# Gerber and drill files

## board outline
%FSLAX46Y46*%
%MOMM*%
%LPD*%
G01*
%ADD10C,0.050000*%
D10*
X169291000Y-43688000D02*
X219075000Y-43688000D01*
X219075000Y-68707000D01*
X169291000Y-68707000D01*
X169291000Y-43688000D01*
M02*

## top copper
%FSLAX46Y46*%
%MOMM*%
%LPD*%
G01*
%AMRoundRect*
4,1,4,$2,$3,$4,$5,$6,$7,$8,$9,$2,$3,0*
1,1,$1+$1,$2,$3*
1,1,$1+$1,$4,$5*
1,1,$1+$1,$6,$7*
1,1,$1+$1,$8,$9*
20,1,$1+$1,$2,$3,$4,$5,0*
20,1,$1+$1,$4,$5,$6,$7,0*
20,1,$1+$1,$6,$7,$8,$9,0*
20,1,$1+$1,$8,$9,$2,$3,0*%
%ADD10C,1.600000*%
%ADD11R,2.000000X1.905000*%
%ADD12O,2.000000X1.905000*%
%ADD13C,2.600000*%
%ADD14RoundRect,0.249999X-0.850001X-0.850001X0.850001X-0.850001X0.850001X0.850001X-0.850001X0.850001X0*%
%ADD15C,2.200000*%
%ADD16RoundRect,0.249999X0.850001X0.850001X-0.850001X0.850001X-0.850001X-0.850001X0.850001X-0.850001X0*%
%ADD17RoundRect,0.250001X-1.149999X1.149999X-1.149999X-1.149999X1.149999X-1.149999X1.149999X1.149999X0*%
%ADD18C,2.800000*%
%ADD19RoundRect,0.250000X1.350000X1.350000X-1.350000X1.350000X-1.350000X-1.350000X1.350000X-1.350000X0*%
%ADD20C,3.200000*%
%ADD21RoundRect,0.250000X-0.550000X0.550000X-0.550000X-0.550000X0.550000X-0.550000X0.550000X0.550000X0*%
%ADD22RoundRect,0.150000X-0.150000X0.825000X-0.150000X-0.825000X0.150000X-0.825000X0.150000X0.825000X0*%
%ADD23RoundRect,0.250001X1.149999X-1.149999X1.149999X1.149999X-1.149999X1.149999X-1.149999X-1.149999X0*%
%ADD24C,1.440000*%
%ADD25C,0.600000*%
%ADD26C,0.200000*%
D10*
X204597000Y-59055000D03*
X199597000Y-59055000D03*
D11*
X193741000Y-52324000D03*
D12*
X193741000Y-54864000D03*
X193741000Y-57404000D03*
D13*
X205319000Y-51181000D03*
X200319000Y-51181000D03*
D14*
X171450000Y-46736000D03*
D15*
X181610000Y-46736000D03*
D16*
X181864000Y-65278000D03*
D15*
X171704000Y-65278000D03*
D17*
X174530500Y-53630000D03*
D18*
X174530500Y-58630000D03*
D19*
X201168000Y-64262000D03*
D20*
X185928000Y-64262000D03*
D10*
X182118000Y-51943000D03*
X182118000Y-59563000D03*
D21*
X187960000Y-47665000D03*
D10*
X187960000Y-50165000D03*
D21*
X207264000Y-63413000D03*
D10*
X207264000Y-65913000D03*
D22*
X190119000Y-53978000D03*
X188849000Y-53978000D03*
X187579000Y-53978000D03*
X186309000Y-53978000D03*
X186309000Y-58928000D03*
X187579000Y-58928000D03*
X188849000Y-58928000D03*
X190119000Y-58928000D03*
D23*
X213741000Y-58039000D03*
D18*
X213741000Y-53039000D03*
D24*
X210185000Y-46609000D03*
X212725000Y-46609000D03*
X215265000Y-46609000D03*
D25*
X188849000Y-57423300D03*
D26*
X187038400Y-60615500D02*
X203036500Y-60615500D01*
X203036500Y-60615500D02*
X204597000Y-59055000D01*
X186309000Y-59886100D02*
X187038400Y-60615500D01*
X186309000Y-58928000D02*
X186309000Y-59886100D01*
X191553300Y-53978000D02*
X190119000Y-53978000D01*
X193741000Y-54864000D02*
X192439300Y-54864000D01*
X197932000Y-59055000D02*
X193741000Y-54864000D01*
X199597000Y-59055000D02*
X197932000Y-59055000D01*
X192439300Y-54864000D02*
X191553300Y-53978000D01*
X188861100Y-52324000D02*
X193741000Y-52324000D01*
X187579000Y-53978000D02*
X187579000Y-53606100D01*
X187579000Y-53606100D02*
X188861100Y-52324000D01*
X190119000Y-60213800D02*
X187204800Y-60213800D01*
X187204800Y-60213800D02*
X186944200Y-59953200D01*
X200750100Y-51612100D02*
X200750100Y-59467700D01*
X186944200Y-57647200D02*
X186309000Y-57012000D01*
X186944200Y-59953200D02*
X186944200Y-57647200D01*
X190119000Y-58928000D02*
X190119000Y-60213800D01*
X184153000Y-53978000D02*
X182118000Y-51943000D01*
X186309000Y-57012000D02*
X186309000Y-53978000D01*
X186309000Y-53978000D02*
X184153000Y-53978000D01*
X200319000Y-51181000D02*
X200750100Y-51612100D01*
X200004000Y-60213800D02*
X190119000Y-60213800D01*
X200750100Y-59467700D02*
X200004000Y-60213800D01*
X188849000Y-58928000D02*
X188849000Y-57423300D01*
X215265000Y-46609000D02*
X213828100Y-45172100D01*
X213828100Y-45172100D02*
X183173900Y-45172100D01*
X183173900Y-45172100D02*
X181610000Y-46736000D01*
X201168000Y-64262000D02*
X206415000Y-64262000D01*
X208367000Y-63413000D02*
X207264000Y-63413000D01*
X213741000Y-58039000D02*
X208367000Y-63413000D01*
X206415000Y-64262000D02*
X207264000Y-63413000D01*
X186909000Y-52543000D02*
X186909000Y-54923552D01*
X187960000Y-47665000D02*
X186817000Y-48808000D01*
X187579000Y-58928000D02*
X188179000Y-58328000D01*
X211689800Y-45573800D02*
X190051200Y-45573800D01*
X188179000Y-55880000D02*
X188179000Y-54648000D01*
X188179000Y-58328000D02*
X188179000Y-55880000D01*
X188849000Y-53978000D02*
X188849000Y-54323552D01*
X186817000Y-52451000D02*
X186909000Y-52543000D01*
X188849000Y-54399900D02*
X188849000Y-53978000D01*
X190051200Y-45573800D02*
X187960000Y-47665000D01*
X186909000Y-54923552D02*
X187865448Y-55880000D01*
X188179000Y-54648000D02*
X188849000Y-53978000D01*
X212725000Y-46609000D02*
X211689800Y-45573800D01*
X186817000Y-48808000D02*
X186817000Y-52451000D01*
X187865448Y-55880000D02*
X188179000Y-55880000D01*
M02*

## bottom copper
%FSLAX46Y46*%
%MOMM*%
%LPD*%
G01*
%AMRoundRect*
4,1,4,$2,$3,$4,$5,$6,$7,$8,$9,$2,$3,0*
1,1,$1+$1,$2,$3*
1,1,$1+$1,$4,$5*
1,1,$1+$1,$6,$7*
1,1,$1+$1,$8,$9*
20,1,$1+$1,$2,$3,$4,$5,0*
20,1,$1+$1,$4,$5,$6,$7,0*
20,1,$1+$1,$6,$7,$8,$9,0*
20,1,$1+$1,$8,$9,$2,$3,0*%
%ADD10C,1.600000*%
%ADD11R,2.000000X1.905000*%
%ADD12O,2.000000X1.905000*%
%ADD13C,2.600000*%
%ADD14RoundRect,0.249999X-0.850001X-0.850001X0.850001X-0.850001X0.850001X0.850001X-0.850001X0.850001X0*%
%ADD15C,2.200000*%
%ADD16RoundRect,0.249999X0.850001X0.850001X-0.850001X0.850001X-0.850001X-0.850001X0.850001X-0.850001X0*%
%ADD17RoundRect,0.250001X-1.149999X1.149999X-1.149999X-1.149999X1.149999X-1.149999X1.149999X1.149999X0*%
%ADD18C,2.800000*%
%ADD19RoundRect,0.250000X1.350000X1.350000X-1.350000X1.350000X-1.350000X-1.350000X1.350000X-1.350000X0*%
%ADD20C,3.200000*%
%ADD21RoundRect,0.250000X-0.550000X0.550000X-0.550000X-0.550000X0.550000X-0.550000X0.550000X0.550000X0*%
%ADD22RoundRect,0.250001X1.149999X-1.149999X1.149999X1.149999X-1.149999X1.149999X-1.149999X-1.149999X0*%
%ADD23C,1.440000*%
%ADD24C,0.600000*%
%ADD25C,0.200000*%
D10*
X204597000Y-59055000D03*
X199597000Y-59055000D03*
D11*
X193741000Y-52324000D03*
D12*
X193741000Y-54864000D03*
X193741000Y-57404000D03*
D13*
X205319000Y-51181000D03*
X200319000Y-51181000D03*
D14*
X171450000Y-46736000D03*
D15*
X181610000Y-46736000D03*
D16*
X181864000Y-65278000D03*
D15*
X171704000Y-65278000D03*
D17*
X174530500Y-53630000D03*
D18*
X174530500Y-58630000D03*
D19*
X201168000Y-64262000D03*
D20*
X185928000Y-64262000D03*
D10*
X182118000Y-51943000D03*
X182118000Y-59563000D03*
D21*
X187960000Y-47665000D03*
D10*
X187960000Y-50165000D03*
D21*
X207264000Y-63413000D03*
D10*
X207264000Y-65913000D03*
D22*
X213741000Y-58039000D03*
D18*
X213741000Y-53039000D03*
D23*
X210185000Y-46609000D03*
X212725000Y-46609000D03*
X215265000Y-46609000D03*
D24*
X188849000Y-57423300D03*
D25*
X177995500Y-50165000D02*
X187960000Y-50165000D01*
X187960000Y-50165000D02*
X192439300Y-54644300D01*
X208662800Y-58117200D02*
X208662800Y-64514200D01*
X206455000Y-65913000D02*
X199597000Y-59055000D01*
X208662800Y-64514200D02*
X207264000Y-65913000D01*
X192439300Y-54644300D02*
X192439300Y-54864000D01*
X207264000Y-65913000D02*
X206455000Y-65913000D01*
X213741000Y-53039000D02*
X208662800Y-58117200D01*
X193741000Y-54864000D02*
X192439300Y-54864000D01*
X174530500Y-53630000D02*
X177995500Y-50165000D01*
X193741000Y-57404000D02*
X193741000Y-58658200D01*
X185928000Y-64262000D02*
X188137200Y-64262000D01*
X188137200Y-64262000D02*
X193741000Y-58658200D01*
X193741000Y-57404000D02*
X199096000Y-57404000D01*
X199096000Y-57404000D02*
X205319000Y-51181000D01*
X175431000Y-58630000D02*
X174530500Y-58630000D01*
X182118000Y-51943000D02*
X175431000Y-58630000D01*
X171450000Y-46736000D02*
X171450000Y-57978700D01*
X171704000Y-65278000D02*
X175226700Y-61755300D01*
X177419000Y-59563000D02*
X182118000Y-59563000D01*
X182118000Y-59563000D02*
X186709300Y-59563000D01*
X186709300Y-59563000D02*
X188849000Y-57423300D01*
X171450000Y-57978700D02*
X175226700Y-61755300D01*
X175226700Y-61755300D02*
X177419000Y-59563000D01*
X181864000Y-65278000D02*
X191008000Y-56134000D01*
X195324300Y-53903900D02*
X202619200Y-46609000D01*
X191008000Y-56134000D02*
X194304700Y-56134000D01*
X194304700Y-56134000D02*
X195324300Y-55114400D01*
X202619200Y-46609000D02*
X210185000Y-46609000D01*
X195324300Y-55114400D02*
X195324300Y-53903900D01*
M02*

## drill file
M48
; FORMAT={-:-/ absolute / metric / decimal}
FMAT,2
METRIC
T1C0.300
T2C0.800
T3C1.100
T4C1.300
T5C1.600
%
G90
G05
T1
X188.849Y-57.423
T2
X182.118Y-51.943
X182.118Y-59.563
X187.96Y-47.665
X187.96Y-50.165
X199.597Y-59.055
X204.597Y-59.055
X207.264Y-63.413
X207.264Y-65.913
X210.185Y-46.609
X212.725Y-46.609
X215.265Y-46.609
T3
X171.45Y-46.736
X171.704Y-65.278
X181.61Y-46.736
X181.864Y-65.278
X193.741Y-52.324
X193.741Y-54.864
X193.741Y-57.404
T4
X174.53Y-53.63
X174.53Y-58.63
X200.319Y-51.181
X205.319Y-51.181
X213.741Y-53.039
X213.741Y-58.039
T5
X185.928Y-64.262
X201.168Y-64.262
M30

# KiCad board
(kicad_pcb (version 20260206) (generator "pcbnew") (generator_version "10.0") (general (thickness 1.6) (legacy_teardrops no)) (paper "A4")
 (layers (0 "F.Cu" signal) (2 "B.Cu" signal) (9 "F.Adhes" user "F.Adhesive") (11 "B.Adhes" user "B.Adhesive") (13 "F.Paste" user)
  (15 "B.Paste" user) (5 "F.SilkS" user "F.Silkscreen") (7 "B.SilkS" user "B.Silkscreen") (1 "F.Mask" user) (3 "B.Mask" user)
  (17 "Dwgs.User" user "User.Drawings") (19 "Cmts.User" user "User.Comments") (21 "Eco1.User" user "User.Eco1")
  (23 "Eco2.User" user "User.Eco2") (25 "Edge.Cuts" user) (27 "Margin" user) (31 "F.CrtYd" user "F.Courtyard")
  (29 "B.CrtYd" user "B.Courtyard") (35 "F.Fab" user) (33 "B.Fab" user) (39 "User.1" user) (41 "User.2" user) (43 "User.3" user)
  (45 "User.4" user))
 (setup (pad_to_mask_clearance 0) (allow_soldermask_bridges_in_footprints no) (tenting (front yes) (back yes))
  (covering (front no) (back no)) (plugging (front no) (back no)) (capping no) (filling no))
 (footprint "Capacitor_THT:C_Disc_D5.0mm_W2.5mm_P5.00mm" (layer "F.Cu") (at 204.597 59.055 180)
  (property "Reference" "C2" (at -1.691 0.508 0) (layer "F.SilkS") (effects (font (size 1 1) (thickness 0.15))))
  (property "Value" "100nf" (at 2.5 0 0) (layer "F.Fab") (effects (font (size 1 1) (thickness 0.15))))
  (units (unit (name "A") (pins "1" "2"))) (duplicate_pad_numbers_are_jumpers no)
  (pad "1" thru_hole circle (at 0 0 180) (size 1.6 1.6) (drill 0.8) (layers "*.Cu" "*.Mask") (remove_unused_layers no) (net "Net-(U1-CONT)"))
  (pad "2" thru_hole circle (at 5 0 180) (size 1.6 1.6) (drill 0.8) (layers "*.Cu" "*.Mask") (remove_unused_layers no) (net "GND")))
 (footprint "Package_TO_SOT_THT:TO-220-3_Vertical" (layer "F.Cu") (at 193.741 52.324 -90)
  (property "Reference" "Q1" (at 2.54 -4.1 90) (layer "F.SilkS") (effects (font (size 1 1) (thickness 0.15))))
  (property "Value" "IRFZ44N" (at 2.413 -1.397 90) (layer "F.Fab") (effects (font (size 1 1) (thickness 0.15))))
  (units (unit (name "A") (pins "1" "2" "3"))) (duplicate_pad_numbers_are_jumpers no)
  (pad "1" thru_hole rect (at 0 0 270) (size 1.905 2) (drill 1.1) (layers "*.Cu" "*.Mask") (remove_unused_layers no) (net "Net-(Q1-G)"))
  (pad "2" thru_hole oval (at 2.54 0 270) (size 1.905 2) (drill 1.1) (layers "*.Cu" "*.Mask") (remove_unused_layers no) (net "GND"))
  (pad "3" thru_hole oval (at 5.08 0 270) (size 1.905 2) (drill 1.1) (layers "*.Cu" "*.Mask") (remove_unused_layers no) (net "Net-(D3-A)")))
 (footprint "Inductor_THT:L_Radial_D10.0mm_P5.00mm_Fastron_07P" (layer "F.Cu") (at 205.319 51.181 180)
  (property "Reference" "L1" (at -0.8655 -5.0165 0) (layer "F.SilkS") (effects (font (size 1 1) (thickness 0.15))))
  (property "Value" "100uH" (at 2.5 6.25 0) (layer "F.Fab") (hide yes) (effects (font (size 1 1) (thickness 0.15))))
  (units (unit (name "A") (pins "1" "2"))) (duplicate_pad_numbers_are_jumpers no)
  (pad "1" thru_hole circle (at 0 0 180) (size 2.6 2.6) (drill 1.3) (layers "*.Cu" "*.Mask") (remove_unused_layers no) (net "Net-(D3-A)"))
  (pad "2" thru_hole circle (at 5 0 180) (size 2.6 2.6) (drill 1.3) (layers "*.Cu" "*.Mask") (remove_unused_layers no)
   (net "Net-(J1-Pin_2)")))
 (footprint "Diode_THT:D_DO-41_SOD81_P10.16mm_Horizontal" (layer "F.Cu") (at 171.45 46.736)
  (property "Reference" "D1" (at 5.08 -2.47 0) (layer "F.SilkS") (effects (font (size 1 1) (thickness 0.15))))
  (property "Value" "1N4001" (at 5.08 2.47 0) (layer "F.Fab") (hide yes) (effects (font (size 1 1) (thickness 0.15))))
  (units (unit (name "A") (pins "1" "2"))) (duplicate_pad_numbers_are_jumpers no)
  (pad "1" thru_hole roundrect (at 0 0) (size 2.2 2.2) (drill 1.1) (layers "*.Cu" "*.Mask") (remove_unused_layers no)
   (roundrect_rratio 0.113636) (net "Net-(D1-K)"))
  (pad "2" thru_hole circle (at 10.16 0) (size 2.2 2.2) (drill 1.1) (layers "*.Cu" "*.Mask") (remove_unused_layers no) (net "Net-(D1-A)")))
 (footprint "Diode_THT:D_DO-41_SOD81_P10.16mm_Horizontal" (layer "F.Cu") (at 181.864 65.278 180)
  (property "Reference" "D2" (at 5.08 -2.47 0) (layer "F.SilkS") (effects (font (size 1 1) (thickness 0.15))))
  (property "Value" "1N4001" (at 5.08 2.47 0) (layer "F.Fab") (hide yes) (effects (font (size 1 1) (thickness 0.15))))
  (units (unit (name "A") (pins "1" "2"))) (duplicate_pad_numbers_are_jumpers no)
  (pad "1" thru_hole roundrect (at 0 0 180) (size 2.2 2.2) (drill 1.1) (layers "*.Cu" "*.Mask") (remove_unused_layers no)
   (roundrect_rratio 0.113636) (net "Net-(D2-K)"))
  (pad "2" thru_hole circle (at 10.16 0 180) (size 2.2 2.2) (drill 1.1) (layers "*.Cu" "*.Mask") (remove_unused_layers no)
   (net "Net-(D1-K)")))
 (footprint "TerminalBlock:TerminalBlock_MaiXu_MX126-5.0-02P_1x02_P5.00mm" (layer "F.Cu") (at 174.5305 53.63 -90)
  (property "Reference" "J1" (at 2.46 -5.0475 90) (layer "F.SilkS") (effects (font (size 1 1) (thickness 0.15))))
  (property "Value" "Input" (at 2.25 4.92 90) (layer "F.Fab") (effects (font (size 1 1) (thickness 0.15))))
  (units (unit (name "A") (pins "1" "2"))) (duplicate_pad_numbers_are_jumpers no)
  (pad "1" thru_hole roundrect (at 0 0 270) (size 2.8 2.8) (drill 1.3) (layers "*.Cu" "*.Mask") (remove_unused_layers no)
   (roundrect_rratio 0.089286) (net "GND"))
  (pad "2" thru_hole circle (at 5 0 270) (size 2.8 2.8) (drill 1.3) (layers "*.Cu" "*.Mask") (remove_unused_layers no)
   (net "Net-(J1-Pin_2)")))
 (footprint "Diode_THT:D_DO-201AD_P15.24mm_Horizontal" (layer "F.Cu") (at 201.168 64.262 180)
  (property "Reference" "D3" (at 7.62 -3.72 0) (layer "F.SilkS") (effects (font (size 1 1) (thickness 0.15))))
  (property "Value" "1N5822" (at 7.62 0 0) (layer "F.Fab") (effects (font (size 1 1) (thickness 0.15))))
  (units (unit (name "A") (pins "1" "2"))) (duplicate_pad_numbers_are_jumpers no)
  (pad "1" thru_hole roundrect (at 0 0 180) (size 3.2 3.2) (drill 1.6) (layers "*.Cu" "*.Mask") (remove_unused_layers no)
   (roundrect_rratio 0.078125) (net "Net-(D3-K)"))
  (pad "2" thru_hole circle (at 15.24 0 180) (size 3.2 3.2) (drill 1.6) (layers "*.Cu" "*.Mask") (remove_unused_layers no)
   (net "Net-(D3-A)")))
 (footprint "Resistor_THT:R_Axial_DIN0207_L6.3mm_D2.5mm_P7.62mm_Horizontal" (layer "F.Cu") (at 182.118 51.943 -90)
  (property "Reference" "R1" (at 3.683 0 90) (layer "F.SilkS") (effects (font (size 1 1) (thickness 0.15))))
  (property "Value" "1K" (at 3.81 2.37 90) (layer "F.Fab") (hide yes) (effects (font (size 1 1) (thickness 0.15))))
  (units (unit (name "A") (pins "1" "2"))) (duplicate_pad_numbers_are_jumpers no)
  (pad "1" thru_hole circle (at 0 0 270) (size 1.6 1.6) (drill 0.8) (layers "*.Cu" "*.Mask") (remove_unused_layers no)
   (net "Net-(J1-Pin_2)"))
  (pad "2" thru_hole circle (at 7.62 0 270) (size 1.6 1.6) (drill 0.8) (layers "*.Cu" "*.Mask") (remove_unused_layers no) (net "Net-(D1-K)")))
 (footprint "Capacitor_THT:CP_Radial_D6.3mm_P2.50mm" (layer "F.Cu") (at 187.96 47.665 -90)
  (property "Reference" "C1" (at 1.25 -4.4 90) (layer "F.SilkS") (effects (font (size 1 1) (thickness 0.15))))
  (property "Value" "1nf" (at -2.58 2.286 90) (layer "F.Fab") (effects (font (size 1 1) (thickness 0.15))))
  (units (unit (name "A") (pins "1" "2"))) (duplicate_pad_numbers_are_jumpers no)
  (pad "1" thru_hole roundrect (at 0 0 270) (size 1.6 1.6) (drill 0.8) (layers "*.Cu" "*.Mask") (remove_unused_layers no)
   (roundrect_rratio 0.15625) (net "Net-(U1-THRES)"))
  (pad "2" thru_hole circle (at 2.5 0 270) (size 1.6 1.6) (drill 0.8) (layers "*.Cu" "*.Mask") (remove_unused_layers no) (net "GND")))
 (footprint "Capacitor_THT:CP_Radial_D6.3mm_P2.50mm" (layer "F.Cu") (at 207.264 63.413 -90)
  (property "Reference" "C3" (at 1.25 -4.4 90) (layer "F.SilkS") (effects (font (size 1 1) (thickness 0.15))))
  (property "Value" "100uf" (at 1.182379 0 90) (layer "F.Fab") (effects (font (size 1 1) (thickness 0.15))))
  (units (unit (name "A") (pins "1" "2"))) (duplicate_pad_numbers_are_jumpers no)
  (pad "1" thru_hole roundrect (at 0 0 270) (size 1.6 1.6) (drill 0.8) (layers "*.Cu" "*.Mask") (remove_unused_layers no)
   (roundrect_rratio 0.15625) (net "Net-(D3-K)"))
  (pad "2" thru_hole circle (at 2.5 0 270) (size 1.6 1.6) (drill 0.8) (layers "*.Cu" "*.Mask") (remove_unused_layers no) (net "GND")))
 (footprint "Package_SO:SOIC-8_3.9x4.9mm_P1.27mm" (layer "F.Cu") (at 188.214 56.453 -90)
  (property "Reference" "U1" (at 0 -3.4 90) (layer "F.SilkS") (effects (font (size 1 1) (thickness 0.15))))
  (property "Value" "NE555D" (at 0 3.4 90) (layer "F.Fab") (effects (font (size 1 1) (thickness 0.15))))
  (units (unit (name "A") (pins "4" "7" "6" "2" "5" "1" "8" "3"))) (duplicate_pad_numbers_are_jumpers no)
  (pad "1" smd roundrect (at -2.475 -1.905 270) (size 1.95 0.6) (layers "F.Cu" "F.Mask" "F.Paste") (roundrect_rratio 0.25) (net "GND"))
  (pad "2" smd roundrect (at -2.475 -0.635 270) (size 1.95 0.6) (layers "F.Cu" "F.Mask" "F.Paste") (roundrect_rratio 0.25)
   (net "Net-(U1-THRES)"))
  (pad "3" smd roundrect (at -2.475 0.635 270) (size 1.95 0.6) (layers "F.Cu" "F.Mask" "F.Paste") (roundrect_rratio 0.25) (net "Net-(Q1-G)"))
  (pad "4" smd roundrect (at -2.475 1.905 270) (size 1.95 0.6) (layers "F.Cu" "F.Mask" "F.Paste") (roundrect_rratio 0.25)
   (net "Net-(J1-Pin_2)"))
  (pad "5" smd roundrect (at 2.475 1.905 270) (size 1.95 0.6) (layers "F.Cu" "F.Mask" "F.Paste") (roundrect_rratio 0.25)
   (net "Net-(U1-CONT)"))
  (pad "6" smd roundrect (at 2.475 0.635 270) (size 1.95 0.6) (layers "F.Cu" "F.Mask" "F.Paste") (roundrect_rratio 0.25)
   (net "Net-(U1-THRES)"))
  (pad "7" smd roundrect (at 2.475 -0.635 270) (size 1.95 0.6) (layers "F.Cu" "F.Mask" "F.Paste") (roundrect_rratio 0.25) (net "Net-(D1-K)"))
  (pad "8" smd roundrect (at 2.475 -1.905 270) (size 1.95 0.6) (layers "F.Cu" "F.Mask" "F.Paste") (roundrect_rratio 0.25)
   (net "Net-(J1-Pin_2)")))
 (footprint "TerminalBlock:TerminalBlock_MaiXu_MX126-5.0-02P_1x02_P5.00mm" (layer "F.Cu") (at 213.741 58.039 90)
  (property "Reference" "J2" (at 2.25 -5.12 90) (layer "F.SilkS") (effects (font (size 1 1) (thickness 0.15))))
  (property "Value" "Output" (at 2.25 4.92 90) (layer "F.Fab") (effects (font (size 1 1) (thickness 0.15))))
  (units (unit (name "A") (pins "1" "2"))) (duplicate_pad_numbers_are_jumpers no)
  (pad "1" thru_hole roundrect (at 0 0 90) (size 2.8 2.8) (drill 1.3) (layers "*.Cu" "*.Mask") (remove_unused_layers no)
   (roundrect_rratio 0.089286) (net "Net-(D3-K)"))
  (pad "2" thru_hole circle (at 5 0 90) (size 2.8 2.8) (drill 1.3) (layers "*.Cu" "*.Mask") (remove_unused_layers no) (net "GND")))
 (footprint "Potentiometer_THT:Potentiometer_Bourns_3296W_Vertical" (layer "F.Cu") (at 210.185 46.609 180)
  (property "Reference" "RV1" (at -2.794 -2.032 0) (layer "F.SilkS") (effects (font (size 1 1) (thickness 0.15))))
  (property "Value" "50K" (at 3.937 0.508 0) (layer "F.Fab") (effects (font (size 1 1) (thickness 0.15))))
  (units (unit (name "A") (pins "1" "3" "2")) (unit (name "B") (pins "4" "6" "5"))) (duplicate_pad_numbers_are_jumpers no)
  (pad "1" thru_hole circle (at 0 0 180) (size 1.44 1.44) (drill 0.8) (layers "*.Cu" "*.Mask") (remove_unused_layers no) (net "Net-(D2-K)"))
  (pad "2" thru_hole circle (at -2.54 0 180) (size 1.44 1.44) (drill 0.8) (layers "*.Cu" "*.Mask") (remove_unused_layers no)
   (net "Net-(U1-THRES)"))
  (pad "3" thru_hole circle (at -5.08 0 180) (size 1.44 1.44) (drill 0.8) (layers "*.Cu" "*.Mask") (remove_unused_layers no)
   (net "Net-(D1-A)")))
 (gr_rect (start 169.291 43.688) (end 219.075 68.707) (stroke (width 0.05) (type default)) (fill no) (layer "Edge.Cuts"))
 (segment (start 187.0384 60.6155) (end 203.0365 60.6155) (width 0.2) (layer "F.Cu") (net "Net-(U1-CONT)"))
 (segment (start 203.0365 60.6155) (end 204.597 59.055) (width 0.2) (layer "F.Cu") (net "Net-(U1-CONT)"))
 (segment (start 186.309 59.8861) (end 187.0384 60.6155) (width 0.2) (layer "F.Cu") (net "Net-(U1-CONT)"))
 (segment (start 186.309 58.928) (end 186.309 59.8861) (width 0.2) (layer "F.Cu") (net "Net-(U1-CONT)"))
 (segment (start 191.5533 53.978) (end 190.119 53.978) (width 0.2) (layer "F.Cu") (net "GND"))
 (segment (start 193.741 54.864) (end 192.4393 54.864) (width 0.2) (layer "F.Cu") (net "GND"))
 (segment (start 197.932 59.055) (end 193.741 54.864) (width 0.2) (layer "F.Cu") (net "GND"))
 (segment (start 199.597 59.055) (end 197.932 59.055) (width 0.2) (layer "F.Cu") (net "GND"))
 (segment (start 192.4393 54.864) (end 191.5533 53.978) (width 0.2) (layer "F.Cu") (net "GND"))
 (segment (start 177.9955 50.165) (end 187.96 50.165) (width 0.2) (layer "B.Cu") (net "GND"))
 (segment (start 187.96 50.165) (end 192.4393 54.6443) (width 0.2) (layer "B.Cu") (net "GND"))
 (segment (start 208.6628 58.1172) (end 208.6628 64.5142) (width 0.2) (layer "B.Cu") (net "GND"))
 (segment (start 206.455 65.913) (end 199.597 59.055) (width 0.2) (layer "B.Cu") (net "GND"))
 (segment (start 208.6628 64.5142) (end 207.264 65.913) (width 0.2) (layer "B.Cu") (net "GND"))
 (segment (start 192.4393 54.6443) (end 192.4393 54.864) (width 0.2) (layer "B.Cu") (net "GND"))
 (segment (start 207.264 65.913) (end 206.455 65.913) (width 0.2) (layer "B.Cu") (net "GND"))
 (segment (start 213.741 53.039) (end 208.6628 58.1172) (width 0.2) (layer "B.Cu") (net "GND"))
 (segment (start 193.741 54.864) (end 192.4393 54.864) (width 0.2) (layer "B.Cu") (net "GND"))
 (segment (start 174.5305 53.63) (end 177.9955 50.165) (width 0.2) (layer "B.Cu") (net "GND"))
 (segment (start 188.8611 52.324) (end 193.741 52.324) (width 0.2) (layer "F.Cu") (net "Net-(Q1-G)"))
 (segment (start 187.579 53.978) (end 187.579 53.6061) (width 0.2) (layer "F.Cu") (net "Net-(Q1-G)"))
 (segment (start 187.579 53.6061) (end 188.8611 52.324) (width 0.2) (layer "F.Cu") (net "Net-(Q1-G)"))
 (segment (start 193.741 57.404) (end 193.741 58.6582) (width 0.2) (layer "B.Cu") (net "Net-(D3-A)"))
 (segment (start 185.928 64.262) (end 188.1372 64.262) (width 0.2) (layer "B.Cu") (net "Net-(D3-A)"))
 (segment (start 188.1372 64.262) (end 193.741 58.6582) (width 0.2) (layer "B.Cu") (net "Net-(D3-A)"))
 (segment (start 193.741 57.404) (end 199.096 57.404) (width 0.2) (layer "B.Cu") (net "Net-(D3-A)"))
 (segment (start 199.096 57.404) (end 205.319 51.181) (width 0.2) (layer "B.Cu") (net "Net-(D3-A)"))
 (segment (start 190.119 60.2138) (end 187.2048 60.2138) (width 0.2) (layer "F.Cu") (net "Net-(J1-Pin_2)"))
 (segment (start 187.2048 60.2138) (end 186.9442 59.9532) (width 0.2) (layer "F.Cu") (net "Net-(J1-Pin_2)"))
 (segment (start 200.7501 51.6121) (end 200.7501 59.4677) (width 0.2) (layer "F.Cu") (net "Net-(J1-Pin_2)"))
 (segment (start 186.9442 57.6472) (end 186.309 57.012) (width 0.2) (layer "F.Cu") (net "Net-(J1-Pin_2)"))
 (segment (start 186.9442 59.9532) (end 186.9442 57.6472) (width 0.2) (layer "F.Cu") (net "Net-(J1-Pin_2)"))
 (segment (start 190.119 58.928) (end 190.119 60.2138) (width 0.2) (layer "F.Cu") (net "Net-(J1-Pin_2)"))
 (segment (start 184.153 53.978) (end 182.118 51.943) (width 0.2) (layer "F.Cu") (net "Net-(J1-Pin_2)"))
 (segment (start 186.309 57.012) (end 186.309 53.978) (width 0.2) (layer "F.Cu") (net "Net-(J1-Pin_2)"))
 (segment (start 186.309 53.978) (end 184.153 53.978) (width 0.2) (layer "F.Cu") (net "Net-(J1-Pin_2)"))
 (segment (start 200.319 51.181) (end 200.7501 51.6121) (width 0.2) (layer "F.Cu") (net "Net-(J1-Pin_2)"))
 (segment (start 200.004 60.2138) (end 190.119 60.2138) (width 0.2) (layer "F.Cu") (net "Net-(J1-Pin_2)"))
 (segment (start 200.7501 59.4677) (end 200.004 60.2138) (width 0.2) (layer "F.Cu") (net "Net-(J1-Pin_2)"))
 (segment (start 175.431 58.63) (end 174.5305 58.63) (width 0.2) (layer "B.Cu") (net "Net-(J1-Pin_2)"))
 (segment (start 182.118 51.943) (end 175.431 58.63) (width 0.2) (layer "B.Cu") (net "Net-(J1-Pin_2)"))
 (segment (start 188.849 58.928) (end 188.849 57.4233) (width 0.2) (layer "F.Cu") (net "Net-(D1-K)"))
 (via (at 188.849 57.4233) (size 0.6) (drill 0.3) (layers "F.Cu" "B.Cu") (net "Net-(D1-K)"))
 (segment (start 171.45 46.736) (end 171.45 57.9787) (width 0.2) (layer "B.Cu") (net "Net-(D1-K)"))
 (segment (start 171.704 65.278) (end 175.2267 61.7553) (width 0.2) (layer "B.Cu") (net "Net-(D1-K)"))
 (segment (start 177.419 59.563) (end 182.118 59.563) (width 0.2) (layer "B.Cu") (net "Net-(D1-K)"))
 (segment (start 182.118 59.563) (end 186.7093 59.563) (width 0.2) (layer "B.Cu") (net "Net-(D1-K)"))
 (segment (start 186.7093 59.563) (end 188.849 57.4233) (width 0.2) (layer "B.Cu") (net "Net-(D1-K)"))
 (segment (start 171.45 57.9787) (end 175.2267 61.7553) (width 0.2) (layer "B.Cu") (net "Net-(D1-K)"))
 (segment (start 175.2267 61.7553) (end 177.419 59.563) (width 0.2) (layer "B.Cu") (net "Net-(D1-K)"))
 (segment (start 215.265 46.609) (end 213.8281 45.1721) (width 0.2) (layer "F.Cu") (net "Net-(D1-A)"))
 (segment (start 213.8281 45.1721) (end 183.1739 45.1721) (width 0.2) (layer "F.Cu") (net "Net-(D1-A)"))
 (segment (start 183.1739 45.1721) (end 181.61 46.736) (width 0.2) (layer "F.Cu") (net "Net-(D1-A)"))
 (segment (start 181.864 65.278) (end 191.008 56.134) (width 0.2) (layer "B.Cu") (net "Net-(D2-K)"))
 (segment (start 195.3243 53.9039) (end 202.6192 46.609) (width 0.2) (layer "B.Cu") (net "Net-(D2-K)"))
 (segment (start 191.008 56.134) (end 194.3047 56.134) (width 0.2) (layer "B.Cu") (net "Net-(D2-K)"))
 (segment (start 194.3047 56.134) (end 195.3243 55.1144) (width 0.2) (layer "B.Cu") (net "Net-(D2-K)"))
 (segment (start 202.6192 46.609) (end 210.185 46.609) (width 0.2) (layer "B.Cu") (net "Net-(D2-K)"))
 (segment (start 195.3243 55.1144) (end 195.3243 53.9039) (width 0.2) (layer "B.Cu") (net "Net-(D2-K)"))
 (segment (start 201.168 64.262) (end 206.415 64.262) (width 0.2) (layer "F.Cu") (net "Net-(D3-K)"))
 (segment (start 208.367 63.413) (end 207.264 63.413) (width 0.2) (layer "F.Cu") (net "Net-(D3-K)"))
 (segment (start 213.741 58.039) (end 208.367 63.413) (width 0.2) (layer "F.Cu") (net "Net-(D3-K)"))
 (segment (start 206.415 64.262) (end 207.264 63.413) (width 0.2) (layer "F.Cu") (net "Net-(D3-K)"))
 (segment (start 186.909 52.543) (end 186.909 54.923552) (width 0.2) (layer "F.Cu") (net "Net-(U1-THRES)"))
 (segment (start 187.96 47.665) (end 186.817 48.808) (width 0.2) (layer "F.Cu") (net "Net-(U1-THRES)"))
 (segment (start 187.579 58.928) (end 188.179 58.328) (width 0.2) (layer "F.Cu") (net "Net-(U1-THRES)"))
 (segment (start 211.6898 45.5738) (end 190.0512 45.5738) (width 0.2) (layer "F.Cu") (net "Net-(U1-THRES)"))
 (segment (start 188.179 55.88) (end 188.179 54.648) (width 0.2) (layer "F.Cu") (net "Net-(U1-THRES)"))
 (segment (start 188.179 58.328) (end 188.179 55.88) (width 0.2) (layer "F.Cu") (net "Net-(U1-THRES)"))
 (segment (start 188.849 53.978) (end 188.849 54.323552) (width 0.2) (layer "F.Cu") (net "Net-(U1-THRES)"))
 (segment (start 186.817 52.451) (end 186.909 52.543) (width 0.2) (layer "F.Cu") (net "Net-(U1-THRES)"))
 (segment (start 188.849 54.3999) (end 188.849 53.978) (width 0.2) (layer "F.Cu") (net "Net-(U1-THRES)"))
 (segment (start 190.0512 45.5738) (end 187.96 47.665) (width 0.2) (layer "F.Cu") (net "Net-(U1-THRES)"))
 (segment (start 186.909 54.923552) (end 187.865448 55.88) (width 0.2) (layer "F.Cu") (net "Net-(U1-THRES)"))
 (segment (start 188.179 54.648) (end 188.849 53.978) (width 0.2) (layer "F.Cu") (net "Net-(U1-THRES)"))
 (segment (start 212.725 46.609) (end 211.6898 45.5738) (width 0.2) (layer "F.Cu") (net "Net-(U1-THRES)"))
 (segment (start 186.817 48.808) (end 186.817 52.451) (width 0.2) (layer "F.Cu") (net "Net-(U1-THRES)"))
 (segment (start 187.865448 55.88) (end 188.179 55.88) (width 0.2) (layer "F.Cu") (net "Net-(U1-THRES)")))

